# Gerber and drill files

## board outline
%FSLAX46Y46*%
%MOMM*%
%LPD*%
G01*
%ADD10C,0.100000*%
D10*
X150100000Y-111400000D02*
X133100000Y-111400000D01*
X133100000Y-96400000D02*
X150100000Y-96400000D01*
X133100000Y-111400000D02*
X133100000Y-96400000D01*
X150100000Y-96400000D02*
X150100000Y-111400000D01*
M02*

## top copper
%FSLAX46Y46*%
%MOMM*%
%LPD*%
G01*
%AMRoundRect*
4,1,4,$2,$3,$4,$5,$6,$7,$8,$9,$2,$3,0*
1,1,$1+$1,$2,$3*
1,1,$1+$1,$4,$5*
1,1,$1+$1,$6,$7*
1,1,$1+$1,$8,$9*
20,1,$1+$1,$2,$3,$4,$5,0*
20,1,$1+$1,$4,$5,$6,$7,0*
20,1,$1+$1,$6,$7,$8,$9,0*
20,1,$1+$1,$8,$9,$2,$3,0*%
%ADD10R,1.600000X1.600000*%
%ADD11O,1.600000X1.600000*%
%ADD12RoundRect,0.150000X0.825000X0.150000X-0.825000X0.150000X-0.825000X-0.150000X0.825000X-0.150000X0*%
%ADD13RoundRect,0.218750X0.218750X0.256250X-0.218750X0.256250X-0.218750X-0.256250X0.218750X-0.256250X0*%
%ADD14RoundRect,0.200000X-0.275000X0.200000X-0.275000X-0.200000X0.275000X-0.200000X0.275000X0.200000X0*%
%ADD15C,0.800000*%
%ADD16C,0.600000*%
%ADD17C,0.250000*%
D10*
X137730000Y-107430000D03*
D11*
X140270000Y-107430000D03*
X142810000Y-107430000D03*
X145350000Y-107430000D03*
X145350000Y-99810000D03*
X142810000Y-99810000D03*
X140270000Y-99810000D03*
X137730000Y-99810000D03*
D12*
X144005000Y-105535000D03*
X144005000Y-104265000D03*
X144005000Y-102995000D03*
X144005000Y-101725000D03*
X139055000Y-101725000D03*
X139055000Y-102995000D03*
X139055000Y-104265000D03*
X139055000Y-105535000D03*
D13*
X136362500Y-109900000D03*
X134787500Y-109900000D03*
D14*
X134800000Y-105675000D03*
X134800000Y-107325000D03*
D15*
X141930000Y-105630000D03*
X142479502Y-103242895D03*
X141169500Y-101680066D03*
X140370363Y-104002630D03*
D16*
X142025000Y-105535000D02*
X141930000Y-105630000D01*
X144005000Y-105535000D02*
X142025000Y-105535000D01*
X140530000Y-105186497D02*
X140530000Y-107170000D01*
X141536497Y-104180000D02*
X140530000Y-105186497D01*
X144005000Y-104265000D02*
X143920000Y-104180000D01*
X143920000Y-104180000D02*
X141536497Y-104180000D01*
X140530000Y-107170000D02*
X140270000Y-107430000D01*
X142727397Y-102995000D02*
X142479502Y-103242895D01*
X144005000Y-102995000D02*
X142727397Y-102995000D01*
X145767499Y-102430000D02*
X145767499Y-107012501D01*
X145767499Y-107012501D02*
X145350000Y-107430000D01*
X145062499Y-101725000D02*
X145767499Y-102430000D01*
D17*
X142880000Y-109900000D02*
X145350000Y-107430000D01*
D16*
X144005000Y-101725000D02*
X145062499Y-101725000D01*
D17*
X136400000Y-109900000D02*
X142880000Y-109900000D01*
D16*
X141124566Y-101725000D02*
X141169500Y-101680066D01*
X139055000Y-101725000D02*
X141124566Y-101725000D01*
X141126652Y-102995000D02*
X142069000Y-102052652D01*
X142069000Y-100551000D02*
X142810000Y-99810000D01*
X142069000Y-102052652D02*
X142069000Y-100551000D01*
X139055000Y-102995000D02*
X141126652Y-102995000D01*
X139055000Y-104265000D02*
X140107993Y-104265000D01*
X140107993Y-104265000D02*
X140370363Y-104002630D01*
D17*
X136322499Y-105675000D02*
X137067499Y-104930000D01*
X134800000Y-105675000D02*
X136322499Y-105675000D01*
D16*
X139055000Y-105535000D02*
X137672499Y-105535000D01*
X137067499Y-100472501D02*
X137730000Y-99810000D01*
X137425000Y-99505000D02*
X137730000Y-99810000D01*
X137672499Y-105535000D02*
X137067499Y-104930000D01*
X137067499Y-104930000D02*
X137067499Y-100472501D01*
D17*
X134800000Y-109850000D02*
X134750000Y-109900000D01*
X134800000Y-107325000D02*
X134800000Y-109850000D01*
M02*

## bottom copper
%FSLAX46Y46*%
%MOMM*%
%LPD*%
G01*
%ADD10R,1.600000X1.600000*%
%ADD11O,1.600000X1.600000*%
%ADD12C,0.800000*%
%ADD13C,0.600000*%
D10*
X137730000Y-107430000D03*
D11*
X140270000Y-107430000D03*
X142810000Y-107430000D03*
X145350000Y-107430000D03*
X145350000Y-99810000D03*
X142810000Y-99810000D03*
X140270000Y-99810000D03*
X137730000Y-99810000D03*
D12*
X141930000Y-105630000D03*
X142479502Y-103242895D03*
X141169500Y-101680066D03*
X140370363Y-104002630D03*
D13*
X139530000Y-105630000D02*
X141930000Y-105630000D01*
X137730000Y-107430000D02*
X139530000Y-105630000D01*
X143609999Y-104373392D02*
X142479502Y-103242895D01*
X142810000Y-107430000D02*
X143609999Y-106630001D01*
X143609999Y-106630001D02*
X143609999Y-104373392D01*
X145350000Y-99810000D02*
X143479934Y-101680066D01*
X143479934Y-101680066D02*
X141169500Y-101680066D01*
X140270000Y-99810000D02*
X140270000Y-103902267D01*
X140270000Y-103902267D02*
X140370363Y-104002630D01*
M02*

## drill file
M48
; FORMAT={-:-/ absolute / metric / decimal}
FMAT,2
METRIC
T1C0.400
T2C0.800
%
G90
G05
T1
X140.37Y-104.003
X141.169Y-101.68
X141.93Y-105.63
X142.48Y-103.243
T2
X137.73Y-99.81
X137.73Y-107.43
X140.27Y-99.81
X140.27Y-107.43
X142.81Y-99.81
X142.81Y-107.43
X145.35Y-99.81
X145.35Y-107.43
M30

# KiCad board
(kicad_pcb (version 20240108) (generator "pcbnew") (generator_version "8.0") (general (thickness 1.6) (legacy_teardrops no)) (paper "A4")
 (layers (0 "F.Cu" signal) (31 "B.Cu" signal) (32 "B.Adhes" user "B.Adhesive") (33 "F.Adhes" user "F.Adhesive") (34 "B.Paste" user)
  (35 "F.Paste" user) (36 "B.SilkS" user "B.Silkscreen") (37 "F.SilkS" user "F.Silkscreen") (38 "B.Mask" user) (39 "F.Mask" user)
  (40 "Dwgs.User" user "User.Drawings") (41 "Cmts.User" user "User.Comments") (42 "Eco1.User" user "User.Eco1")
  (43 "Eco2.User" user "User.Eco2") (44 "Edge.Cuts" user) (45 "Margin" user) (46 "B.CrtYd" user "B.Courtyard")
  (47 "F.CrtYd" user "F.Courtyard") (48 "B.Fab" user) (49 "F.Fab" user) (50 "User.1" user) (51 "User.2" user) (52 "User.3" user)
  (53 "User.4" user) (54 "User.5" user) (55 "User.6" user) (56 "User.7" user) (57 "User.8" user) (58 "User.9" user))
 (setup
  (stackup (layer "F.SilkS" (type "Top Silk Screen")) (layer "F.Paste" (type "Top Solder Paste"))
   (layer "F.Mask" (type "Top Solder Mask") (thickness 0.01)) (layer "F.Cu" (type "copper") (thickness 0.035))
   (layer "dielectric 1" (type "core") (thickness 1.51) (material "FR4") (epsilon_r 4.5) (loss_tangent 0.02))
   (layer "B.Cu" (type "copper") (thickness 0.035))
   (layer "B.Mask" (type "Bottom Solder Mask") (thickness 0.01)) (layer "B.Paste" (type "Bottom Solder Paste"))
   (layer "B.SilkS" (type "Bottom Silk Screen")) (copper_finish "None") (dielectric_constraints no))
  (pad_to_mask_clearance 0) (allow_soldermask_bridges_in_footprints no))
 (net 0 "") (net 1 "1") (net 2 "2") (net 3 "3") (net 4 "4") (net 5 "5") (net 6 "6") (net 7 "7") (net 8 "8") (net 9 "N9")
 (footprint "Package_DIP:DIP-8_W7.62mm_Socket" (layer "F.Cu") (at 137.73 107.43 90)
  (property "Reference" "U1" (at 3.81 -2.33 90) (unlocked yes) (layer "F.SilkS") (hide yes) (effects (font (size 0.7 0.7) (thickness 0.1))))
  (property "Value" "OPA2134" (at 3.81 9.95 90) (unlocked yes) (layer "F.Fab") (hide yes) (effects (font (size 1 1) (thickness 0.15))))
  (pad "1" thru_hole rect (at 0 0 90) (size 1.6 1.6) (drill 0.8) (layers "*.Cu" "*.Mask") (remove_unused_layers no) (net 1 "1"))
  (pad "2" thru_hole oval (at 0 2.54 90) (size 1.6 1.6) (drill 0.8) (layers "*.Cu" "*.Mask") (remove_unused_layers no) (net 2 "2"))
  (pad "3" thru_hole oval (at 0 5.08 90) (size 1.6 1.6) (drill 0.8) (layers "*.Cu" "*.Mask") (remove_unused_layers no) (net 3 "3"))
  (pad "4" thru_hole oval (at 0 7.62 90) (size 1.6 1.6) (drill 0.8) (layers "*.Cu" "*.Mask") (remove_unused_layers no) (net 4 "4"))
  (pad "5" thru_hole oval (at 7.62 7.62 90) (size 1.6 1.6) (drill 0.8) (layers "*.Cu" "*.Mask") (remove_unused_layers no) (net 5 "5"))
  (pad "6" thru_hole oval (at 7.62 5.08 90) (size 1.6 1.6) (drill 0.8) (layers "*.Cu" "*.Mask") (remove_unused_layers no) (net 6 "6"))
  (pad "7" thru_hole oval (at 7.62 2.54 90) (size 1.6 1.6) (drill 0.8) (layers "*.Cu" "*.Mask") (remove_unused_layers no) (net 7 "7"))
  (pad "8" thru_hole oval (at 7.62 0 90) (size 1.6 1.6) (drill 0.8) (layers "*.Cu" "*.Mask") (remove_unused_layers no) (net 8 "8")))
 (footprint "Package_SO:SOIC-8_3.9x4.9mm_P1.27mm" (layer "F.Cu") (at 141.53 103.63 180)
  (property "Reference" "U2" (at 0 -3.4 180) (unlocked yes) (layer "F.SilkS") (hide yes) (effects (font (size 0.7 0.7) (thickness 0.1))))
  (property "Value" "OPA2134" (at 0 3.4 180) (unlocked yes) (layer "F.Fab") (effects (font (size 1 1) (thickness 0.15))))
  (pad "1" smd roundrect (at -2.475 -1.905 180) (size 1.95 0.6) (layers "F.Cu" "F.Paste" "F.Mask") (roundrect_rratio 0.25) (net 1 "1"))
  (pad "2" smd roundrect (at -2.475 -0.635 180) (size 1.95 0.6) (layers "F.Cu" "F.Paste" "F.Mask") (roundrect_rratio 0.25) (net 2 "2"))
  (pad "3" smd roundrect (at -2.475 0.635 180) (size 1.95 0.6) (layers "F.Cu" "F.Paste" "F.Mask") (roundrect_rratio 0.25) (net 3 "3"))
  (pad "4" smd roundrect (at -2.475 1.905 180) (size 1.95 0.6) (layers "F.Cu" "F.Paste" "F.Mask") (roundrect_rratio 0.25) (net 4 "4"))
  (pad "5" smd roundrect (at 2.475 1.905 180) (size 1.95 0.6) (layers "F.Cu" "F.Paste" "F.Mask") (roundrect_rratio 0.25) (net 5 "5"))
  (pad "6" smd roundrect (at 2.475 0.635 180) (size 1.95 0.6) (layers "F.Cu" "F.Paste" "F.Mask") (roundrect_rratio 0.25) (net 6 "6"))
  (pad "7" smd roundrect (at 2.475 -0.635 180) (size 1.95 0.6) (layers "F.Cu" "F.Paste" "F.Mask") (roundrect_rratio 0.25) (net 7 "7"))
  (pad "8" smd roundrect (at 2.475 -1.905 180) (size 1.95 0.6) (layers "F.Cu" "F.Paste" "F.Mask") (roundrect_rratio 0.25) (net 8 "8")))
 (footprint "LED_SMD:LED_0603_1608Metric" (layer "F.Cu") (at 135.575 109.9 180)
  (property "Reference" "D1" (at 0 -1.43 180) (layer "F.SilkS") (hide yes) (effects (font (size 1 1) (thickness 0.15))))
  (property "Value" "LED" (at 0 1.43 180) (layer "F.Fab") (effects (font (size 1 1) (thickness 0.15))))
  (pad "1" smd roundrect (at -0.7875 0 180) (size 0.875 0.95) (layers "F.Cu" "F.Paste" "F.Mask") (roundrect_rratio 0.25) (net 4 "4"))
  (pad "2" smd roundrect (at 0.7875 0 180) (size 0.875 0.95) (layers "F.Cu" "F.Paste" "F.Mask") (roundrect_rratio 0.25) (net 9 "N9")))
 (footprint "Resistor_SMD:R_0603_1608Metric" (layer "F.Cu") (at 134.8 106.5 -90)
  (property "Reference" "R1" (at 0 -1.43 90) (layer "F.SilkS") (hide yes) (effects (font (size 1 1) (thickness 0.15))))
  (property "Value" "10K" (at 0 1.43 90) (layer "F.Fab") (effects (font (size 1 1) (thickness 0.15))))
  (pad "1" smd roundrect (at -0.825 0 270) (size 0.8 0.95) (layers "F.Cu" "F.Paste" "F.Mask") (roundrect_rratio 0.25) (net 8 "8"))
  (pad "2" smd roundrect (at 0.825 0 270) (size 0.8 0.95) (layers "F.Cu" "F.Paste" "F.Mask") (roundrect_rratio 0.25) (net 9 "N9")))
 (gr_line (start 150.1 111.4) (end 133.1 111.4) (stroke (width 0.1) (type default)) (layer "Edge.Cuts"))
 (gr_line (start 133.1 96.4) (end 150.1 96.4) (stroke (width 0.1) (type default)) (layer "Edge.Cuts"))
 (gr_line (start 133.1 111.4) (end 133.1 96.4) (stroke (width 0.1) (type default)) (layer "Edge.Cuts"))
 (gr_line (start 150.1 96.4) (end 150.1 111.4) (stroke (width 0.1) (type default)) (layer "Edge.Cuts"))
 (segment (start 142.025 105.535) (end 141.93 105.63) (width 0.6) (layer "F.Cu") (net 1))
 (segment (start 144.005 105.535) (end 142.025 105.535) (width 0.6) (layer "F.Cu") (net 1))
 (via (at 141.93 105.63) (size 0.8) (drill 0.4) (layers "F.Cu" "B.Cu") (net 1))
 (segment (start 139.53 105.63) (end 141.93 105.63) (width 0.6) (layer "B.Cu") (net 1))
 (segment (start 137.73 107.43) (end 139.53 105.63) (width 0.6) (layer "B.Cu") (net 1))
 (segment (start 140.53 105.186497) (end 140.53 107.17) (width 0.6) (layer "F.Cu") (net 2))
 (segment (start 141.536497 104.18) (end 140.53 105.186497) (width 0.6) (layer "F.Cu") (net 2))
 (segment (start 144.005 104.265) (end 143.92 104.18) (width 0.6) (layer "F.Cu") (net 2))
 (segment (start 143.92 104.18) (end 141.536497 104.18) (width 0.6) (layer "F.Cu") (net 2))
 (segment (start 140.53 107.17) (end 140.27 107.43) (width 0.6) (layer "F.Cu") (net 2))
 (segment (start 142.727397 102.995) (end 142.479502 103.242895) (width 0.6) (layer "F.Cu") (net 3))
 (segment (start 144.005 102.995) (end 142.727397 102.995) (width 0.6) (layer "F.Cu") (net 3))
 (via (at 142.479502 103.242895) (size 0.8) (drill 0.4) (layers "F.Cu" "B.Cu") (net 3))
 (segment (start 143.609999 104.373392) (end 142.479502 103.242895) (width 0.6) (layer "B.Cu") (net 3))
 (segment (start 142.81 107.43) (end 143.609999 106.630001) (width 0.6) (layer "B.Cu") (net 3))
 (segment (start 143.609999 106.630001) (end 143.609999 104.373392) (width 0.6) (layer "B.Cu") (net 3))
 (segment (start 145.767499 102.43) (end 145.767499 107.012501) (width 0.6) (layer "F.Cu") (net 4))
 (segment (start 145.767499 107.012501) (end 145.35 107.43) (width 0.6) (layer "F.Cu") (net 4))
 (segment (start 145.062499 101.725) (end 145.767499 102.43) (width 0.6) (layer "F.Cu") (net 4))
 (segment (start 142.88 109.9) (end 145.35 107.43) (width 0.25) (layer "F.Cu") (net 4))
 (segment (start 144.005 101.725) (end 145.062499 101.725) (width 0.6) (layer "F.Cu") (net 4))
 (segment (start 136.4 109.9) (end 142.88 109.9) (width 0.25) (layer "F.Cu") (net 4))
 (segment (start 141.124566 101.725) (end 141.1695 101.680066) (width 0.6) (layer "F.Cu") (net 5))
 (segment (start 139.055 101.725) (end 141.124566 101.725) (width 0.6) (layer "F.Cu") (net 5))
 (via (at 141.1695 101.680066) (size 0.8) (drill 0.4) (layers "F.Cu" "B.Cu") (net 5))
 (segment (start 145.35 99.81) (end 143.479934 101.680066) (width 0.6) (layer "B.Cu") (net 5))
 (segment (start 143.479934 101.680066) (end 141.1695 101.680066) (width 0.6) (layer "B.Cu") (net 5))
 (segment (start 141.126652 102.995) (end 142.069 102.052652) (width 0.6) (layer "F.Cu") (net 6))
 (segment (start 142.069 100.551) (end 142.81 99.81) (width 0.6) (layer "F.Cu") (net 6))
 (segment (start 142.069 102.052652) (end 142.069 100.551) (width 0.6) (layer "F.Cu") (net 6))
 (segment (start 139.055 102.995) (end 141.126652 102.995) (width 0.6) (layer "F.Cu") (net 6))
 (segment (start 139.055 104.265) (end 140.107993 104.265) (width 0.6) (layer "F.Cu") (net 7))
 (segment (start 140.107993 104.265) (end 140.370363 104.00263) (width 0.6) (layer "F.Cu") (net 7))
 (via (at 140.370363 104.00263) (size 0.8) (drill 0.4) (layers "F.Cu" "B.Cu") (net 7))
 (segment (start 140.27 99.81) (end 140.27 103.902267) (width 0.6) (layer "B.Cu") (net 7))
 (segment (start 140.27 103.902267) (end 140.370363 104.00263) (width 0.6) (layer "B.Cu") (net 7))
 (segment (start 136.322499 105.675) (end 137.067499 104.93) (width 0.25) (layer "F.Cu") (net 8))
 (segment (start 134.8 105.675) (end 136.322499 105.675) (width 0.25) (layer "F.Cu") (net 8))
 (segment (start 139.055 105.535) (end 137.672499 105.535) (width 0.6) (layer "F.Cu") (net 8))
 (segment (start 137.067499 100.472501) (end 137.73 99.81) (width 0.6) (layer "F.Cu") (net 8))
 (segment (start 137.425 99.505) (end 137.73 99.81) (width 0.6) (layer "F.Cu") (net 8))
 (segment (start 137.672499 105.535) (end 137.067499 104.93) (width 0.6) (layer "F.Cu") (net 8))
 (segment (start 137.067499 104.93) (end 137.067499 100.472501) (width 0.6) (layer "F.Cu") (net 8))
 (segment (start 134.8 109.85) (end 134.75 109.9) (width 0.25) (layer "F.Cu") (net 9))
 (segment (start 134.8 107.325) (end 134.8 109.85) (width 0.25) (layer "F.Cu") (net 9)))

